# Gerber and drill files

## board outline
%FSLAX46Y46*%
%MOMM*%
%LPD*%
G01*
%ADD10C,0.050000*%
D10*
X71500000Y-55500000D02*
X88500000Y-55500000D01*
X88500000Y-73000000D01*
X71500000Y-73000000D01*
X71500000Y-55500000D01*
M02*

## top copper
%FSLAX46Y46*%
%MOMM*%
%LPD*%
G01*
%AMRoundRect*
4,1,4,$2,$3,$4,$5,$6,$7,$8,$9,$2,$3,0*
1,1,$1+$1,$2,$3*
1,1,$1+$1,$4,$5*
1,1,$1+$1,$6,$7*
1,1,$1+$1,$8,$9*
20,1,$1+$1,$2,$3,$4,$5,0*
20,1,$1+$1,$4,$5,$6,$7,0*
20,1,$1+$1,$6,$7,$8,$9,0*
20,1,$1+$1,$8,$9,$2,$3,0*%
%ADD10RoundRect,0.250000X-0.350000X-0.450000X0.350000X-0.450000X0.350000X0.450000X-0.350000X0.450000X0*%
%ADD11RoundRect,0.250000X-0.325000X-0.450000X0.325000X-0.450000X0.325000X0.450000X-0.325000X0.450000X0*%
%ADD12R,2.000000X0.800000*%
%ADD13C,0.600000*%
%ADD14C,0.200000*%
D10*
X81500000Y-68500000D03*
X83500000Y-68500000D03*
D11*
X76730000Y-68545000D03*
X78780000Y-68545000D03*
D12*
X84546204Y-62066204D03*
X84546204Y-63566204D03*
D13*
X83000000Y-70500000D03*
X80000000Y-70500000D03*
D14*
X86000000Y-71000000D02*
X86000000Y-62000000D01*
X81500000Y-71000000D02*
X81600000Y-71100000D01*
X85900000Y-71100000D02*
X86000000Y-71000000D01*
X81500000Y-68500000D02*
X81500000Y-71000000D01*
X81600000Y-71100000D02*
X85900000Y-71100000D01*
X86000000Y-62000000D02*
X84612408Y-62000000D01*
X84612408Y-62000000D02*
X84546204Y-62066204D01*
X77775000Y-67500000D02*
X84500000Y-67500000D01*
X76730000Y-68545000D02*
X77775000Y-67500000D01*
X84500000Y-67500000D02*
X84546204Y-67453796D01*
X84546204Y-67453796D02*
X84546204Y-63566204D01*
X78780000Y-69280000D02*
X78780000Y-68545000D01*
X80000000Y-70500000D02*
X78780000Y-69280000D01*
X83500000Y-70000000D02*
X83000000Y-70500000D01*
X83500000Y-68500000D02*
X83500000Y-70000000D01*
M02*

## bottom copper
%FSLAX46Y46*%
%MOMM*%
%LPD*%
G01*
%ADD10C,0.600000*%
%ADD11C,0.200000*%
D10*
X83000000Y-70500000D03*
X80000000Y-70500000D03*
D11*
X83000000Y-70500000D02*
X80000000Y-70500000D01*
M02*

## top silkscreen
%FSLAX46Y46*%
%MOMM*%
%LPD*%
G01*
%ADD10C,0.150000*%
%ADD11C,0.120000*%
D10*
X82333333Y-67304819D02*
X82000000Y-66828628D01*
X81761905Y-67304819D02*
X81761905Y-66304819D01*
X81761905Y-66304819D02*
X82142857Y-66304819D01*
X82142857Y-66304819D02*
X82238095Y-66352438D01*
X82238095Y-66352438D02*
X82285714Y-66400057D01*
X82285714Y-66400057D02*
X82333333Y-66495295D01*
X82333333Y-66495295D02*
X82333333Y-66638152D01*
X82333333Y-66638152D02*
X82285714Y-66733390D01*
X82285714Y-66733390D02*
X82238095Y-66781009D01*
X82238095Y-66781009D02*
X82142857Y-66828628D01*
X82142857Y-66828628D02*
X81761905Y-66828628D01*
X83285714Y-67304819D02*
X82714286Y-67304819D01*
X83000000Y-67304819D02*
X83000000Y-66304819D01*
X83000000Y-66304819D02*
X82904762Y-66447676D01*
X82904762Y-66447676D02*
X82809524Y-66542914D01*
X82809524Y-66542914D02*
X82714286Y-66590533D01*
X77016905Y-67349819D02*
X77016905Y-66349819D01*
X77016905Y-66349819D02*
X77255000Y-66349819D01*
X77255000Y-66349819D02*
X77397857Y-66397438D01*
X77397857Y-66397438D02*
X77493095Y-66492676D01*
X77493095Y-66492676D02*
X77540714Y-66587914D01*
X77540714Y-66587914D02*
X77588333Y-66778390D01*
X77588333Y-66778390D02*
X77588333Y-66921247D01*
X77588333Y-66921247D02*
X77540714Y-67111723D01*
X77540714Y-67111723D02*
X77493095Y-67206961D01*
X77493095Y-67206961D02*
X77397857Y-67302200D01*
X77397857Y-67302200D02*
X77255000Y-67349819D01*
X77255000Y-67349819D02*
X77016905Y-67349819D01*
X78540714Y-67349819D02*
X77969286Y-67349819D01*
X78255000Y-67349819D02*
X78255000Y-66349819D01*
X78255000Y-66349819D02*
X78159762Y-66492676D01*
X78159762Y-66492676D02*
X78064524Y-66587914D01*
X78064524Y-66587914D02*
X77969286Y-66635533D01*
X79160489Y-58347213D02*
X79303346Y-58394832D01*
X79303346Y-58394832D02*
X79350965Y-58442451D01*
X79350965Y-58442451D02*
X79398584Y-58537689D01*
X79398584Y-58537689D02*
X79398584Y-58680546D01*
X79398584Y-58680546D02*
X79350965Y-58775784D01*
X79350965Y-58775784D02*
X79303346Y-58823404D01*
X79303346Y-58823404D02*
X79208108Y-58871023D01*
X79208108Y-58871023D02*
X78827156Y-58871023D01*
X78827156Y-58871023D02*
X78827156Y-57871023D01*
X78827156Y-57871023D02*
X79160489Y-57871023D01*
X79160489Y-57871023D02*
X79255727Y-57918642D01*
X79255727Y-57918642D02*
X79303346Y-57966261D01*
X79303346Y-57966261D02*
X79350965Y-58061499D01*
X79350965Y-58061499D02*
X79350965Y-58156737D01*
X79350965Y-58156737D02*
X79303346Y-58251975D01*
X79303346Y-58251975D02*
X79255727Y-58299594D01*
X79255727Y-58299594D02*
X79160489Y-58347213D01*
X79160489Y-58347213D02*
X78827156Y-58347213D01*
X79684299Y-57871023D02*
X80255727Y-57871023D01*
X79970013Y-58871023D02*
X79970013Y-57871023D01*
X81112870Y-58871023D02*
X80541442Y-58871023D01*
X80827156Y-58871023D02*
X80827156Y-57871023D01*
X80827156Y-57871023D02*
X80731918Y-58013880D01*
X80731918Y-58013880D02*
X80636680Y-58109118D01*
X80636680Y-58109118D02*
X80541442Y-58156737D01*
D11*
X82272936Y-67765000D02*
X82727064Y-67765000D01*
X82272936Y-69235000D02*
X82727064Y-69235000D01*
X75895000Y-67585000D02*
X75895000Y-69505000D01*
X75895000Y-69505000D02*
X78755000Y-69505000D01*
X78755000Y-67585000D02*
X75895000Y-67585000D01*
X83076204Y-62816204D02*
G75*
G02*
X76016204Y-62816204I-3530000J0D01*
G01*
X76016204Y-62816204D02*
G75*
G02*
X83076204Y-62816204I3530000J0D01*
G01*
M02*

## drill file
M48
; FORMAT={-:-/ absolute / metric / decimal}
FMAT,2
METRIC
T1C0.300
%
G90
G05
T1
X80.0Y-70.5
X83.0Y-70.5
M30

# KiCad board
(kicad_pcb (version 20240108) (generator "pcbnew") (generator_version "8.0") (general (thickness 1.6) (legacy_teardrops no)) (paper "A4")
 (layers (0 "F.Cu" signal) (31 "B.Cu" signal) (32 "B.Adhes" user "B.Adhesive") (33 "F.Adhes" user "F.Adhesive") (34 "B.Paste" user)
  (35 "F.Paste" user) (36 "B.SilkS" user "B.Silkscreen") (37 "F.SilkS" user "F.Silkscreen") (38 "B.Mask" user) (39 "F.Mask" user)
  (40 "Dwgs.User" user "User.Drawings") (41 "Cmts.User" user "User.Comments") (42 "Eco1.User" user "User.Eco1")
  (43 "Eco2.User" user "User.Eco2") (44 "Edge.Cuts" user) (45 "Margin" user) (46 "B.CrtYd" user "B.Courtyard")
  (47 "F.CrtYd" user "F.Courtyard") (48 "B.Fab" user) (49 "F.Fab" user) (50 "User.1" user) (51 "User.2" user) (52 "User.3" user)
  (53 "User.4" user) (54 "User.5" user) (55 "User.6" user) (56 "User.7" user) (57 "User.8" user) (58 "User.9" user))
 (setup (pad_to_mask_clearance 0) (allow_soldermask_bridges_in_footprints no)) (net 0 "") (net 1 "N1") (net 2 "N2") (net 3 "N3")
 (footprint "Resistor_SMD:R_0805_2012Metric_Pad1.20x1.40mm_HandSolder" (layer "F.Cu") (at 82.5 68.5)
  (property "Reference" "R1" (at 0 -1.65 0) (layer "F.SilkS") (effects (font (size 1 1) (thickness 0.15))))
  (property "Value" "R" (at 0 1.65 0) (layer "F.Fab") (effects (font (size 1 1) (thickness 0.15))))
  (fp_line (start -0.227064 -0.735) (end 0.227064 -0.735) (stroke (width 0.12) (type solid)) (layer "F.SilkS"))
  (fp_line (start -0.227064 0.735) (end 0.227064 0.735) (stroke (width 0.12) (type solid)) (layer "F.SilkS"))
  (pad "1" smd roundrect (at -1 0) (size 1.2 1.4) (layers "F.Cu" "F.Paste" "F.Mask") (roundrect_rratio 0.208333) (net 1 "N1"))
  (pad "2" smd roundrect (at 1 0) (size 1.2 1.4) (layers "F.Cu" "F.Paste" "F.Mask") (roundrect_rratio 0.208333) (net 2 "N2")))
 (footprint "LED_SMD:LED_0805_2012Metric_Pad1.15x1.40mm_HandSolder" (layer "F.Cu") (at 77.755 68.545)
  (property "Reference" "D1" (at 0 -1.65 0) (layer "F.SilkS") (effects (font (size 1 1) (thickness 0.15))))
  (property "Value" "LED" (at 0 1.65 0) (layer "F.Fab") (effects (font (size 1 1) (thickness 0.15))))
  (fp_line (start -1.86 -0.96) (end -1.86 0.96) (stroke (width 0.12) (type solid)) (layer "F.SilkS"))
  (fp_line (start -1.86 0.96) (end 1 0.96) (stroke (width 0.12) (type solid)) (layer "F.SilkS"))
  (fp_line (start 1 -0.96) (end -1.86 -0.96) (stroke (width 0.12) (type solid)) (layer "F.SilkS"))
  (pad "1" smd roundrect (at -1.025 0) (size 1.15 1.4) (layers "F.Cu" "F.Paste" "F.Mask") (roundrect_rratio 0.217391) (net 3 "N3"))
  (pad "2" smd roundrect (at 1.025 0) (size 1.15 1.4) (layers "F.Cu" "F.Paste" "F.Mask") (roundrect_rratio 0.217391) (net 2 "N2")))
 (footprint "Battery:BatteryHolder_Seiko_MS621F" (layer "F.Cu") (at 84.546204 62.816204)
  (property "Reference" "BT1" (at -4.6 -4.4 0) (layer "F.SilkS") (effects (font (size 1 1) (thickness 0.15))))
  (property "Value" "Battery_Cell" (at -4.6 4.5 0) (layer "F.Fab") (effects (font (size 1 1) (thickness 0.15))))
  (fp_circle (center -5 0) (end -1.47 0) (stroke (width 0.12) (type solid)) (fill none) (layer "F.SilkS"))
  (pad "1" smd rect (at 0 -0.75) (size 2 0.8) (layers "F.Cu" "F.Paste" "F.Mask") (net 1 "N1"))
  (pad "2" smd rect (at 0 0.75) (size 2 0.8) (layers "F.Cu" "F.Paste" "F.Mask") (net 3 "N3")))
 (gr_rect (start 71.5 55.5) (end 88.5 73) (stroke (width 0.05) (type default)) (fill none) (layer "Edge.Cuts"))
 (segment (start 86 71) (end 86 62) (width 0.2) (layer "F.Cu") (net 1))
 (segment (start 81.5 71) (end 81.6 71.1) (width 0.2) (layer "F.Cu") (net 1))
 (segment (start 85.9 71.1) (end 86 71) (width 0.2) (layer "F.Cu") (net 1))
 (segment (start 81.5 68.5) (end 81.5 71) (width 0.2) (layer "F.Cu") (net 1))
 (segment (start 81.6 71.1) (end 85.9 71.1) (width 0.2) (layer "F.Cu") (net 1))
 (segment (start 86 62) (end 84.612408 62) (width 0.2) (layer "F.Cu") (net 1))
 (segment (start 84.612408 62) (end 84.546204 62.066204) (width 0.2) (layer "F.Cu") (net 1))
 (segment (start 77.775 67.5) (end 84.5 67.5) (width 0.2) (layer "F.Cu") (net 3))
 (segment (start 76.73 68.545) (end 77.775 67.5) (width 0.2) (layer "F.Cu") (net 3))
 (segment (start 84.5 67.5) (end 84.546204 67.453796) (width 0.2) (layer "F.Cu") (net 3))
 (segment (start 84.546204 67.453796) (end 84.546204 63.566204) (width 0.2) (layer "F.Cu") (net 3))
 (segment (start 78.78 69.28) (end 78.78 68.545) (width 0.2) (layer "F.Cu") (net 2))
 (segment (start 80 70.5) (end 78.78 69.28) (width 0.2) (layer "F.Cu") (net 2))
 (segment (start 83.5 70) (end 83 70.5) (width 0.2) (layer "F.Cu") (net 2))
 (segment (start 83.5 68.5) (end 83.5 70) (width 0.2) (layer "F.Cu") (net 2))
 (via (at 83 70.5) (size 0.6) (drill 0.3) (layers "F.Cu" "B.Cu") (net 2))
 (via (at 80 70.5) (size 0.6) (drill 0.3) (layers "F.Cu" "B.Cu") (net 2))
 (segment (start 83 70.5) (end 80 70.5) (width 0.2) (layer "B.Cu") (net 2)))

